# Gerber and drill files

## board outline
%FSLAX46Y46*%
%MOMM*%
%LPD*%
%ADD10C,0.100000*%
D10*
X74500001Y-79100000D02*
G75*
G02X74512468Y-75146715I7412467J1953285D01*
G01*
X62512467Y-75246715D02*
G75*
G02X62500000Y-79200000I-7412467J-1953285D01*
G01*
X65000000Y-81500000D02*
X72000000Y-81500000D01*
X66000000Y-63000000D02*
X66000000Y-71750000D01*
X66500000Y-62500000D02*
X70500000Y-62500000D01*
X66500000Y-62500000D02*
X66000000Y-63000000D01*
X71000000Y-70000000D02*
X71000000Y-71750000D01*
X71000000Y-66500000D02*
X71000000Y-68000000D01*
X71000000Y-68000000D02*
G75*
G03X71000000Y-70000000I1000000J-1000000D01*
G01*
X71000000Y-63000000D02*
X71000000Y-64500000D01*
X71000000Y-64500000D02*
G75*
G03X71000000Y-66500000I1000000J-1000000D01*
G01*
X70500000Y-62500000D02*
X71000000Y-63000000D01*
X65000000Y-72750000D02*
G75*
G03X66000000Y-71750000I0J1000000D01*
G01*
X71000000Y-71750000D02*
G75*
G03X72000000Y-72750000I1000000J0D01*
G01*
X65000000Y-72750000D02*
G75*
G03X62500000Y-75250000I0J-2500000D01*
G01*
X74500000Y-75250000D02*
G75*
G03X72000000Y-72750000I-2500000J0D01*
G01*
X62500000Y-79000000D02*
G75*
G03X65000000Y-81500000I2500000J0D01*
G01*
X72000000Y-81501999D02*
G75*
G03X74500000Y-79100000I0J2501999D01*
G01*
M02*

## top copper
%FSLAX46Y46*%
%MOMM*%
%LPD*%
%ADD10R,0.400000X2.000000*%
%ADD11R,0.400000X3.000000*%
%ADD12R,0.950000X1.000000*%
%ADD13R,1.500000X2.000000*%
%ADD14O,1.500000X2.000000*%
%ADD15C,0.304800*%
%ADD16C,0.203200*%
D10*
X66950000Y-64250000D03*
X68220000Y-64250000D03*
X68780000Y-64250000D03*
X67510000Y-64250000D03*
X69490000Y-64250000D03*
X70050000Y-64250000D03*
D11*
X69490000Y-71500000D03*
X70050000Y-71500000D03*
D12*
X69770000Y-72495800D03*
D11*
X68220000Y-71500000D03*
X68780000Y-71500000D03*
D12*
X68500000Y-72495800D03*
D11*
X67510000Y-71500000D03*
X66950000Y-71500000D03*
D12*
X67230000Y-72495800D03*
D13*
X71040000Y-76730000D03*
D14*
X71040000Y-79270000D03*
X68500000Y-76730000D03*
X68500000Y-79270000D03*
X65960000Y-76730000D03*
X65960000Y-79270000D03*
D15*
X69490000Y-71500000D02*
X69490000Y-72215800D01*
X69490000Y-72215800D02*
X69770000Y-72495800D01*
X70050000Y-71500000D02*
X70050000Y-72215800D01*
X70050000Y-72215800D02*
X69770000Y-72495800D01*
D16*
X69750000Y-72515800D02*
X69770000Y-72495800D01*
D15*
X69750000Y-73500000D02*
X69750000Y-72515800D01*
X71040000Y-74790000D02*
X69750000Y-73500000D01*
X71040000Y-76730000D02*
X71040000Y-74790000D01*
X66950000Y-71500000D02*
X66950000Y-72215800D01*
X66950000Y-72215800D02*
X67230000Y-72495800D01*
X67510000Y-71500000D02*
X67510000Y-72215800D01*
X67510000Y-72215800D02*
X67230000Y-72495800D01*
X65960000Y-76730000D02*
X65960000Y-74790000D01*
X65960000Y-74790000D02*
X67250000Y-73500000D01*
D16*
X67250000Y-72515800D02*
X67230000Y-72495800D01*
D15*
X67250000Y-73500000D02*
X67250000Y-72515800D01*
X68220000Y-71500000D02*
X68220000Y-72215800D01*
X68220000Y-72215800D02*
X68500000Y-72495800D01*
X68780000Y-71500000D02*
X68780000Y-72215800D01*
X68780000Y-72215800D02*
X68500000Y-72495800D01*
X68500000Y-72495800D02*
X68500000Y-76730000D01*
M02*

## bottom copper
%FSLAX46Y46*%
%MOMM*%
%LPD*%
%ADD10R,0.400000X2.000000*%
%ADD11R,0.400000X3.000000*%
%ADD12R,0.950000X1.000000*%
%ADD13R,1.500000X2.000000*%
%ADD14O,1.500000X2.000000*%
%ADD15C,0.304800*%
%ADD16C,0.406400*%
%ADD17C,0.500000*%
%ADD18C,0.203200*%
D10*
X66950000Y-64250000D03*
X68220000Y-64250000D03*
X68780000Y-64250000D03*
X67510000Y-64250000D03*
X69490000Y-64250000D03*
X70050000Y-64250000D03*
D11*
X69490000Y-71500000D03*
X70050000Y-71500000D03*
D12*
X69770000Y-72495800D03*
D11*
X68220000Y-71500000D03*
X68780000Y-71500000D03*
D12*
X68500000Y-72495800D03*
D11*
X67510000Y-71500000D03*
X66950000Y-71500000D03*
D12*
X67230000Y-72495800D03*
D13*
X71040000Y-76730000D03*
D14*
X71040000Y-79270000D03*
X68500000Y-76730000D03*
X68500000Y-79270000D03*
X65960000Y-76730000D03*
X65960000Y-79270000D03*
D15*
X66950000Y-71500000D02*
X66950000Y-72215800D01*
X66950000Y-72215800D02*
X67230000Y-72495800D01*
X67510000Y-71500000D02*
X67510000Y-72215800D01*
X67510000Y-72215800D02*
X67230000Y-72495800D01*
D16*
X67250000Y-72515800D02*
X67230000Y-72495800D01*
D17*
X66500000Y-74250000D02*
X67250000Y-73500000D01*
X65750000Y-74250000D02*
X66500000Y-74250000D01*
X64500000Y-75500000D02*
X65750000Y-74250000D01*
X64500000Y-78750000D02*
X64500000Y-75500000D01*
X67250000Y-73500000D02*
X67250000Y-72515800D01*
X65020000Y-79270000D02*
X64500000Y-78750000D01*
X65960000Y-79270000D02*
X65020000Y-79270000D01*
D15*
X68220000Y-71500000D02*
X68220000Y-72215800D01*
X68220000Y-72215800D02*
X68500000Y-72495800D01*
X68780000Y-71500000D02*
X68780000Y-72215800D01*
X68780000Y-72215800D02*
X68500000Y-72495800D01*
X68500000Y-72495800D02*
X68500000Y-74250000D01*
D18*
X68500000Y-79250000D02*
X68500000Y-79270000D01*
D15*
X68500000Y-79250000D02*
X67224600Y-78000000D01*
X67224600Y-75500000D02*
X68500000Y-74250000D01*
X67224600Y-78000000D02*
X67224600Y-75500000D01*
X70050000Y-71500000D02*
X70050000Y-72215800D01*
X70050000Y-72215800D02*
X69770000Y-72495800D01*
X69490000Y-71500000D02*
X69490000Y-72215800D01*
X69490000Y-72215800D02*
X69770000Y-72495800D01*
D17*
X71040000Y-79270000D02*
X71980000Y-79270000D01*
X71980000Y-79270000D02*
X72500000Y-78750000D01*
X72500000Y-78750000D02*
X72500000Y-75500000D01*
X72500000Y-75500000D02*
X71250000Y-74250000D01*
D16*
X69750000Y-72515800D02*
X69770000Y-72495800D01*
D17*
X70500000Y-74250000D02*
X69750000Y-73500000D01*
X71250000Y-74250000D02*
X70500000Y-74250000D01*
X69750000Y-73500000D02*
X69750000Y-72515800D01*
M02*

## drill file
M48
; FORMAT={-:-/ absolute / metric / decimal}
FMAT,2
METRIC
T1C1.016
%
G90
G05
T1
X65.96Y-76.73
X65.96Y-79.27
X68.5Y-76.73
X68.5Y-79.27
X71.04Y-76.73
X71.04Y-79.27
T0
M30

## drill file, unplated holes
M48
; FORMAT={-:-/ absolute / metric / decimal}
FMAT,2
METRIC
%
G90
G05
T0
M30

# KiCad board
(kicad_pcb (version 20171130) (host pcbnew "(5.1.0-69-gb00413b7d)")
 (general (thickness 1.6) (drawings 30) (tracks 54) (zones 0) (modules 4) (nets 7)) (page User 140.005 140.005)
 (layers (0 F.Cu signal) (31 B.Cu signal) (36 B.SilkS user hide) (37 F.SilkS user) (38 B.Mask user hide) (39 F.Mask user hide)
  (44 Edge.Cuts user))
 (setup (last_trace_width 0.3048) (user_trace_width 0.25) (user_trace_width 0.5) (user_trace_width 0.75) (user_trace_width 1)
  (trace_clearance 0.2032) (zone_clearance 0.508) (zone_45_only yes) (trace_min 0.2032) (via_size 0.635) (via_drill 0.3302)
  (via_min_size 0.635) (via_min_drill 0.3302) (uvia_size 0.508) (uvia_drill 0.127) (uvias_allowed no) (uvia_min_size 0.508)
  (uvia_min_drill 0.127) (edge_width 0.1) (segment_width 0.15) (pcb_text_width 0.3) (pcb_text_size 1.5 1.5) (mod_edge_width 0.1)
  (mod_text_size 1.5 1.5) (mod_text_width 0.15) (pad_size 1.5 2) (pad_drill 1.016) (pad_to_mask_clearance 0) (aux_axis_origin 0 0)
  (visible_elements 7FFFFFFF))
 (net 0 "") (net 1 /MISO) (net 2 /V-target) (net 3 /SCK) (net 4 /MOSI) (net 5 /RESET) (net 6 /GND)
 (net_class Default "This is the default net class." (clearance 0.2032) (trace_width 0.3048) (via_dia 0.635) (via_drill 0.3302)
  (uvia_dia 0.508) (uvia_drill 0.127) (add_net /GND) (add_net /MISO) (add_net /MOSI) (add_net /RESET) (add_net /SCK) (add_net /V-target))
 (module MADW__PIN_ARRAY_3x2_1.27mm (layer F.Cu) (at 68.5 68) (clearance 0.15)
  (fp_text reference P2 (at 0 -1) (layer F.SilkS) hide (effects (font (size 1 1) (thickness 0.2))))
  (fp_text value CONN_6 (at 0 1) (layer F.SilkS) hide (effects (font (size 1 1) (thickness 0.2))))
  (pad ~ smd rect (at -1.55 -3.75) (size 0.4 2) (layers F.Cu F.Mask))
  (pad ~ smd rect (at -0.28 -3.75) (size 0.4 2) (layers F.Cu F.Mask))
  (pad ~ smd rect (at 0.28 -3.75) (size 0.4 2) (layers F.Cu F.Mask))
  (pad ~ smd rect (at -0.99 -3.75) (size 0.4 2) (layers F.Cu F.Mask))
  (pad ~ smd rect (at 0.99 -3.75) (size 0.4 2) (layers F.Cu F.Mask))
  (pad ~ smd rect (at 1.55 -3.75) (size 0.4 2) (layers F.Cu F.Mask))
  (pad ~ smd rect (at -1.55 -3.75) (size 0.4 2) (layers B.Cu F.Mask))
  (pad ~ smd rect (at -0.28 -3.75) (size 0.4 2) (layers B.Cu F.Mask))
  (pad ~ smd rect (at 0.28 -3.75) (size 0.4 2) (layers B.Cu F.Mask))
  (pad ~ smd rect (at -0.99 -3.75) (size 0.4 2) (layers B.Cu F.Mask))
  (pad ~ smd rect (at 0.99 -3.75) (size 0.4 2) (layers B.Cu F.Mask))
  (pad ~ smd rect (at 1.55 -3.75) (size 0.4 2) (layers B.Cu F.Mask))
  (pad 1 smd rect (at 0.99 3.5) (size 0.4 3) (layers F.Cu F.Mask) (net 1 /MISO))
  (pad 1 smd rect (at 1.55 3.5) (size 0.4 3) (layers F.Cu F.Mask) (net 1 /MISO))
  (pad 1 smd rect (at 1.27 4.4958) (size 0.95 1) (layers F.Cu F.Mask) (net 1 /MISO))
  (pad 2 smd rect (at 0.99 3.5) (size 0.4 3) (layers B.Cu F.Mask) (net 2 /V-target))
  (pad 2 smd rect (at 1.55 3.5) (size 0.4 3) (layers B.Cu F.Mask) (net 2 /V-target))
  (pad 2 smd rect (at 1.27 4.4958) (size 0.95 1) (layers B.Cu B.Mask) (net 2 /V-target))
  (pad 3 smd rect (at -0.28 3.5) (size 0.4 3) (layers F.Cu F.Mask) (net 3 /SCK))
  (pad 3 smd rect (at 0.28 3.5) (size 0.4 3) (layers F.Cu F.Mask) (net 3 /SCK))
  (pad 3 smd rect (at 0 4.4958) (size 0.95 1) (layers F.Cu F.Mask) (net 3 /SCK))
  (pad 4 smd rect (at -0.28 3.5) (size 0.4 3) (layers B.Cu F.Mask) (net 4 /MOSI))
  (pad 4 smd rect (at 0.28 3.5) (size 0.4 3) (layers B.Cu F.Mask) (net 4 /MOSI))
  (pad 4 smd rect (at 0 4.4958) (size 0.95 1) (layers B.Cu B.Mask) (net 4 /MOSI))
  (pad 5 smd rect (at -0.99 3.5) (size 0.4 3) (layers F.Cu F.Mask) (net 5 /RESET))
  (pad 5 smd rect (at -1.55 3.5) (size 0.4 3) (layers F.Cu F.Mask) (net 5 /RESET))
  (pad 5 smd rect (at -1.27 4.4958) (size 0.95 1) (layers F.Cu F.Mask) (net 5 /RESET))
  (pad 6 smd rect (at -0.99 3.5) (size 0.4 3) (layers B.Cu F.Mask) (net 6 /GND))
  (pad 6 smd rect (at -1.55 3.5) (size 0.4 3) (layers B.Cu F.Mask) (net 6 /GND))
  (pad 6 smd rect (at -1.27 4.4958) (size 0.95 1) (layers B.Cu B.Mask) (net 6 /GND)))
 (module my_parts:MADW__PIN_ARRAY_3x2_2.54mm (layer F.Cu) (at 68.5 78)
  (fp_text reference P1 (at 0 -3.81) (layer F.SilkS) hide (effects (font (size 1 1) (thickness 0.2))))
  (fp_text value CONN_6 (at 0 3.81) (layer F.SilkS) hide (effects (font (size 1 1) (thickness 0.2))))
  (pad 1 thru_hole rect (at 2.54 -1.27) (size 1.5 2) (drill 1.016) (layers *.Cu *.Mask F.SilkS) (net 1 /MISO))
  (pad 2 thru_hole oval (at 2.54 1.27) (size 1.5 2) (drill 1.016) (layers *.Cu *.Mask F.SilkS) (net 2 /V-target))
  (pad 3 thru_hole oval (at 0 -1.27) (size 1.5 2) (drill 1.016) (layers *.Cu *.Mask F.SilkS) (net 3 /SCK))
  (pad 4 thru_hole oval (at 0 1.27) (size 1.5 2) (drill 1.016) (layers *.Cu *.Mask F.SilkS) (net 4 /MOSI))
  (pad 5 thru_hole oval (at -2.54 -1.27) (size 1.5 2) (drill 1.016) (layers *.Cu *.Mask F.SilkS) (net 5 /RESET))
  (pad 6 thru_hole oval (at -2.54 1.27) (size 1.5 2) (drill 1.016) (layers *.Cu *.Mask F.SilkS) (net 6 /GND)))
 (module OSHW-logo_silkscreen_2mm (layer F.Cu) (at 71.95 74.2)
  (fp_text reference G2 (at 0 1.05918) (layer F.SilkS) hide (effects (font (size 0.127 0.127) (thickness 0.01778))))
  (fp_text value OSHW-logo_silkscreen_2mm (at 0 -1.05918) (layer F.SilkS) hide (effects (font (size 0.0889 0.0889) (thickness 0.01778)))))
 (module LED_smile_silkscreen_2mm (layer F.Cu) (at 64.75 74.25)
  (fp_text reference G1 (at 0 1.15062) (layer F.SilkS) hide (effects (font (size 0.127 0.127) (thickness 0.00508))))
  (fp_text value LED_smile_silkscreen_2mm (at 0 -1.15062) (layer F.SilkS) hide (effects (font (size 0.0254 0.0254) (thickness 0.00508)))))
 (gr_arc (start 81.912468 77.146715) (end 74.512468 75.146715) (angle -29.88662428) (layer Edge.Cuts) (width 0.1))
 (gr_arc (start 55.1 77.2) (end 62.5 79.2) (angle -29.88662428) (layer Edge.Cuts) (width 0.1))
 (gr_line (start 65 81.5) (end 72 81.5) (layer Edge.Cuts) (width 0.1))
 (gr_line (start 66 63) (end 66 71.75) (angle 90) (layer Edge.Cuts) (width 0.1))
 (gr_line (start 66.5 62.5) (end 70.5 62.5) (angle 90) (layer Edge.Cuts) (width 0.1))
 (gr_line (start 66.5 62.5) (end 66 63) (angle 90) (layer Edge.Cuts) (width 0.1))
 (gr_line (start 71 70) (end 71 71.75) (angle 90) (layer Edge.Cuts) (width 0.1))
 (gr_line (start 71 66.5) (end 71 68) (angle 90) (layer Edge.Cuts) (width 0.1))
 (gr_arc (start 72 69) (end 71 70) (angle 90) (layer Edge.Cuts) (width 0.1))
 (gr_line (start 71 63) (end 71 64.5) (angle 90) (layer Edge.Cuts) (width 0.1))
 (gr_arc (start 72 65.5) (end 71 66.5) (angle 90) (layer Edge.Cuts) (width 0.1))
 (gr_line (start 70.5 62.5) (end 71 63) (angle 90) (layer Edge.Cuts) (width 0.1))
 (gr_arc (start 65 71.75) (end 66 71.75) (angle 90) (layer Edge.Cuts) (width 0.1))
 (gr_arc (start 72 71.75) (end 72 72.75) (angle 90) (layer Edge.Cuts) (width 0.1))
 (gr_arc (start 65 75.25) (end 62.5 75.25) (angle 90) (layer Edge.Cuts) (width 0.1))
 (gr_arc (start 72 75.25) (end 72 72.75) (angle 90) (layer Edge.Cuts) (width 0.1))
 (gr_arc (start 65 79) (end 65 81.5) (angle 90) (layer Edge.Cuts) (width 0.1))
 (gr_arc (start 72 79) (end 74.5 79) (angle 90) (layer Edge.Cuts) (width 0.1))
 (segment (start 66.95 71.5) (end 66.95 72.2158) (width 0.3048) (layer B.Cu) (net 6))
 (segment (start 66.95 72.2158) (end 67.23 72.4958) (width 0.3048) (layer B.Cu) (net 6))
 (segment (start 67.51 71.5) (end 67.51 72.2158) (width 0.3048) (layer B.Cu) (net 6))
 (segment (start 67.51 72.2158) (end 67.23 72.4958) (width 0.3048) (layer B.Cu) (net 6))
 (segment (start 67.25 72.5158) (end 67.23 72.4958) (width 0.4064) (layer B.Cu) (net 6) (status 30))
 (segment (start 66.5 74.25) (end 67.25 73.5) (width 0.5) (layer B.Cu) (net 6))
 (segment (start 65.75 74.25) (end 66.5 74.25) (width 0.5) (layer B.Cu) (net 6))
 (segment (start 64.5 75.5) (end 65.75 74.25) (width 0.5) (layer B.Cu) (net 6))
 (segment (start 64.5 78.75) (end 64.5 75.5) (width 0.5) (layer B.Cu) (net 6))
 (segment (start 67.25 73.5) (end 67.25 72.5158) (width 0.5) (layer B.Cu) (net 6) (status 20))
 (segment (start 65.02 79.27) (end 64.5 78.75) (width 0.5) (layer B.Cu) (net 6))
 (segment (start 65.96 79.27) (end 65.02 79.27) (width 0.5) (layer B.Cu) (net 6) (status 10))
 (segment (start 69.49 71.5) (end 69.49 72.2158) (width 0.3048) (layer F.Cu) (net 1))
 (segment (start 69.49 72.2158) (end 69.77 72.4958) (width 0.3048) (layer F.Cu) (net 1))
 (segment (start 70.05 71.5) (end 70.05 72.2158) (width 0.3048) (layer F.Cu) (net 1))
 (segment (start 70.05 72.2158) (end 69.77 72.4958) (width 0.3048) (layer F.Cu) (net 1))
 (segment (start 69.75 72.5158) (end 69.77 72.4958) (width 0.2032) (layer F.Cu) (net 1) (status 30))
 (segment (start 69.75 73.5) (end 69.75 72.5158) (width 0.3048) (layer F.Cu) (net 1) (status 20))
 (segment (start 71.04 74.79) (end 69.75 73.5) (width 0.3048) (layer F.Cu) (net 1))
 (segment (start 71.04 76.73) (end 71.04 74.79) (width 0.3048) (layer F.Cu) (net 1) (status 10))
 (segment (start 68.22 71.5) (end 68.22 72.2158) (width 0.3048) (layer B.Cu) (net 4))
 (segment (start 68.22 72.2158) (end 68.5 72.4958) (width 0.3048) (layer B.Cu) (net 4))
 (segment (start 68.78 71.5) (end 68.78 72.2158) (width 0.3048) (layer B.Cu) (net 4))
 (segment (start 68.78 72.2158) (end 68.5 72.4958) (width 0.3048) (layer B.Cu) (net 4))
 (segment (start 68.5 72.4958) (end 68.5 74.25) (width 0.3048) (layer B.Cu) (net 4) (status 10))
 (segment (start 68.5 79.25) (end 68.5 79.27) (width 0.2032) (layer B.Cu) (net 4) (status 30))
 (segment (start 68.5 79.25) (end 67.2246 78) (width 0.3048) (layer B.Cu) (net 4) (status 10))
 (segment (start 67.2246 75.5) (end 68.5 74.25) (width 0.3048) (layer B.Cu) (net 4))
 (segment (start 67.2246 78) (end 67.2246 75.5) (width 0.3048) (layer B.Cu) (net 4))
 (segment (start 66.95 71.5) (end 66.95 72.2158) (width 0.3048) (layer F.Cu) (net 5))
 (segment (start 66.95 72.2158) (end 67.23 72.4958) (width 0.3048) (layer F.Cu) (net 5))
 (segment (start 67.51 71.5) (end 67.51 72.2158) (width 0.3048) (layer F.Cu) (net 5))
 (segment (start 67.51 72.2158) (end 67.23 72.4958) (width 0.3048) (layer F.Cu) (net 5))
 (segment (start 65.96 76.73) (end 65.96 74.79) (width 0.3048) (layer F.Cu) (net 5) (status 10))
 (segment (start 65.96 74.79) (end 67.25 73.5) (width 0.3048) (layer F.Cu) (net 5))
 (segment (start 67.25 72.5158) (end 67.23 72.4958) (width 0.2032) (layer F.Cu) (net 5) (status 30))
 (segment (start 67.25 73.5) (end 67.25 72.5158) (width 0.3048) (layer F.Cu) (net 5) (status 20))
 (segment (start 68.22 71.5) (end 68.22 72.2158) (width 0.3048) (layer F.Cu) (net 3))
 (segment (start 68.22 72.2158) (end 68.5 72.4958) (width 0.3048) (layer F.Cu) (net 3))
 (segment (start 68.78 71.5) (end 68.78 72.2158) (width 0.3048) (layer F.Cu) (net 3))
 (segment (start 68.78 72.2158) (end 68.5 72.4958) (width 0.3048) (layer F.Cu) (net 3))
 (segment (start 68.5 72.4958) (end 68.5 76.73) (width 0.3048) (layer F.Cu) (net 3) (status 30))
 (segment (start 70.05 71.5) (end 70.05 72.2158) (width 0.3048) (layer B.Cu) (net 2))
 (segment (start 70.05 72.2158) (end 69.77 72.4958) (width 0.3048) (layer B.Cu) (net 2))
 (segment (start 69.49 71.5) (end 69.49 72.2158) (width 0.3048) (layer B.Cu) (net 2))
 (segment (start 69.49 72.2158) (end 69.77 72.4958) (width 0.3048) (layer B.Cu) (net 2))
 (segment (start 71.04 79.27) (end 71.98 79.27) (width 0.5) (layer B.Cu) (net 2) (status 10))
 (segment (start 71.98 79.27) (end 72.5 78.75) (width 0.5) (layer B.Cu) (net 2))
 (segment (start 72.5 78.75) (end 72.5 75.5) (width 0.5) (layer B.Cu) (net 2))
 (segment (start 72.5 75.5) (end 71.25 74.25) (width 0.5) (layer B.Cu) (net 2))
 (segment (start 69.75 72.5158) (end 69.77 72.4958) (width 0.4064) (layer B.Cu) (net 2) (status 30))
 (segment (start 70.5 74.25) (end 69.75 73.5) (width 0.5) (layer B.Cu) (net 2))
 (segment (start 71.25 74.25) (end 70.5 74.25) (width 0.5) (layer B.Cu) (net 2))
 (segment (start 69.75 73.5) (end 69.75 72.5158) (width 0.5) (layer B.Cu) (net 2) (status 20))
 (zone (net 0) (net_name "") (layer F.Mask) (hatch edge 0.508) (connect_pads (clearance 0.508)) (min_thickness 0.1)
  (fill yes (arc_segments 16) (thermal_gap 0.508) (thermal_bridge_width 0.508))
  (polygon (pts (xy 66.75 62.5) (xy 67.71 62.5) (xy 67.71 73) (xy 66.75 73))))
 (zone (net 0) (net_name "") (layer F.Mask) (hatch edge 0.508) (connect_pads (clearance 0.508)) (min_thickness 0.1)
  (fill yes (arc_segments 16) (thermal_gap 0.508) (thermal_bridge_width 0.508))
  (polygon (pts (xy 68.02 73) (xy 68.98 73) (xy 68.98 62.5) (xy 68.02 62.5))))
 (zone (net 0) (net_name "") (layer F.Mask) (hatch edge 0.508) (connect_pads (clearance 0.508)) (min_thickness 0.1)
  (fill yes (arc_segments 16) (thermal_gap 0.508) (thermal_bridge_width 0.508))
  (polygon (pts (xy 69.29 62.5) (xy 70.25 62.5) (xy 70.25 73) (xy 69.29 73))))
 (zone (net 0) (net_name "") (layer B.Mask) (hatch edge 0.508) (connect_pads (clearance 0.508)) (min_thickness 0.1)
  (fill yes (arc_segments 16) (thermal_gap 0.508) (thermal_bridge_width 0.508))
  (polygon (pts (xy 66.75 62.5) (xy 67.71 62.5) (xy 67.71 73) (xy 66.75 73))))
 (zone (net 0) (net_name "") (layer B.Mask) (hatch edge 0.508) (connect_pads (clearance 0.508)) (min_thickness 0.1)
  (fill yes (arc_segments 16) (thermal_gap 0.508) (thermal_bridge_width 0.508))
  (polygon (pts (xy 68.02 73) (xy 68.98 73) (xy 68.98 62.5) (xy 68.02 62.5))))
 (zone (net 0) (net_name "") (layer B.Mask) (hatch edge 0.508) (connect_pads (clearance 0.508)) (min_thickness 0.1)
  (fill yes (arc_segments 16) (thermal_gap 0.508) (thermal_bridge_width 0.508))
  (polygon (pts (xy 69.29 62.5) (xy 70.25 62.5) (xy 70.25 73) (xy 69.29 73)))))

